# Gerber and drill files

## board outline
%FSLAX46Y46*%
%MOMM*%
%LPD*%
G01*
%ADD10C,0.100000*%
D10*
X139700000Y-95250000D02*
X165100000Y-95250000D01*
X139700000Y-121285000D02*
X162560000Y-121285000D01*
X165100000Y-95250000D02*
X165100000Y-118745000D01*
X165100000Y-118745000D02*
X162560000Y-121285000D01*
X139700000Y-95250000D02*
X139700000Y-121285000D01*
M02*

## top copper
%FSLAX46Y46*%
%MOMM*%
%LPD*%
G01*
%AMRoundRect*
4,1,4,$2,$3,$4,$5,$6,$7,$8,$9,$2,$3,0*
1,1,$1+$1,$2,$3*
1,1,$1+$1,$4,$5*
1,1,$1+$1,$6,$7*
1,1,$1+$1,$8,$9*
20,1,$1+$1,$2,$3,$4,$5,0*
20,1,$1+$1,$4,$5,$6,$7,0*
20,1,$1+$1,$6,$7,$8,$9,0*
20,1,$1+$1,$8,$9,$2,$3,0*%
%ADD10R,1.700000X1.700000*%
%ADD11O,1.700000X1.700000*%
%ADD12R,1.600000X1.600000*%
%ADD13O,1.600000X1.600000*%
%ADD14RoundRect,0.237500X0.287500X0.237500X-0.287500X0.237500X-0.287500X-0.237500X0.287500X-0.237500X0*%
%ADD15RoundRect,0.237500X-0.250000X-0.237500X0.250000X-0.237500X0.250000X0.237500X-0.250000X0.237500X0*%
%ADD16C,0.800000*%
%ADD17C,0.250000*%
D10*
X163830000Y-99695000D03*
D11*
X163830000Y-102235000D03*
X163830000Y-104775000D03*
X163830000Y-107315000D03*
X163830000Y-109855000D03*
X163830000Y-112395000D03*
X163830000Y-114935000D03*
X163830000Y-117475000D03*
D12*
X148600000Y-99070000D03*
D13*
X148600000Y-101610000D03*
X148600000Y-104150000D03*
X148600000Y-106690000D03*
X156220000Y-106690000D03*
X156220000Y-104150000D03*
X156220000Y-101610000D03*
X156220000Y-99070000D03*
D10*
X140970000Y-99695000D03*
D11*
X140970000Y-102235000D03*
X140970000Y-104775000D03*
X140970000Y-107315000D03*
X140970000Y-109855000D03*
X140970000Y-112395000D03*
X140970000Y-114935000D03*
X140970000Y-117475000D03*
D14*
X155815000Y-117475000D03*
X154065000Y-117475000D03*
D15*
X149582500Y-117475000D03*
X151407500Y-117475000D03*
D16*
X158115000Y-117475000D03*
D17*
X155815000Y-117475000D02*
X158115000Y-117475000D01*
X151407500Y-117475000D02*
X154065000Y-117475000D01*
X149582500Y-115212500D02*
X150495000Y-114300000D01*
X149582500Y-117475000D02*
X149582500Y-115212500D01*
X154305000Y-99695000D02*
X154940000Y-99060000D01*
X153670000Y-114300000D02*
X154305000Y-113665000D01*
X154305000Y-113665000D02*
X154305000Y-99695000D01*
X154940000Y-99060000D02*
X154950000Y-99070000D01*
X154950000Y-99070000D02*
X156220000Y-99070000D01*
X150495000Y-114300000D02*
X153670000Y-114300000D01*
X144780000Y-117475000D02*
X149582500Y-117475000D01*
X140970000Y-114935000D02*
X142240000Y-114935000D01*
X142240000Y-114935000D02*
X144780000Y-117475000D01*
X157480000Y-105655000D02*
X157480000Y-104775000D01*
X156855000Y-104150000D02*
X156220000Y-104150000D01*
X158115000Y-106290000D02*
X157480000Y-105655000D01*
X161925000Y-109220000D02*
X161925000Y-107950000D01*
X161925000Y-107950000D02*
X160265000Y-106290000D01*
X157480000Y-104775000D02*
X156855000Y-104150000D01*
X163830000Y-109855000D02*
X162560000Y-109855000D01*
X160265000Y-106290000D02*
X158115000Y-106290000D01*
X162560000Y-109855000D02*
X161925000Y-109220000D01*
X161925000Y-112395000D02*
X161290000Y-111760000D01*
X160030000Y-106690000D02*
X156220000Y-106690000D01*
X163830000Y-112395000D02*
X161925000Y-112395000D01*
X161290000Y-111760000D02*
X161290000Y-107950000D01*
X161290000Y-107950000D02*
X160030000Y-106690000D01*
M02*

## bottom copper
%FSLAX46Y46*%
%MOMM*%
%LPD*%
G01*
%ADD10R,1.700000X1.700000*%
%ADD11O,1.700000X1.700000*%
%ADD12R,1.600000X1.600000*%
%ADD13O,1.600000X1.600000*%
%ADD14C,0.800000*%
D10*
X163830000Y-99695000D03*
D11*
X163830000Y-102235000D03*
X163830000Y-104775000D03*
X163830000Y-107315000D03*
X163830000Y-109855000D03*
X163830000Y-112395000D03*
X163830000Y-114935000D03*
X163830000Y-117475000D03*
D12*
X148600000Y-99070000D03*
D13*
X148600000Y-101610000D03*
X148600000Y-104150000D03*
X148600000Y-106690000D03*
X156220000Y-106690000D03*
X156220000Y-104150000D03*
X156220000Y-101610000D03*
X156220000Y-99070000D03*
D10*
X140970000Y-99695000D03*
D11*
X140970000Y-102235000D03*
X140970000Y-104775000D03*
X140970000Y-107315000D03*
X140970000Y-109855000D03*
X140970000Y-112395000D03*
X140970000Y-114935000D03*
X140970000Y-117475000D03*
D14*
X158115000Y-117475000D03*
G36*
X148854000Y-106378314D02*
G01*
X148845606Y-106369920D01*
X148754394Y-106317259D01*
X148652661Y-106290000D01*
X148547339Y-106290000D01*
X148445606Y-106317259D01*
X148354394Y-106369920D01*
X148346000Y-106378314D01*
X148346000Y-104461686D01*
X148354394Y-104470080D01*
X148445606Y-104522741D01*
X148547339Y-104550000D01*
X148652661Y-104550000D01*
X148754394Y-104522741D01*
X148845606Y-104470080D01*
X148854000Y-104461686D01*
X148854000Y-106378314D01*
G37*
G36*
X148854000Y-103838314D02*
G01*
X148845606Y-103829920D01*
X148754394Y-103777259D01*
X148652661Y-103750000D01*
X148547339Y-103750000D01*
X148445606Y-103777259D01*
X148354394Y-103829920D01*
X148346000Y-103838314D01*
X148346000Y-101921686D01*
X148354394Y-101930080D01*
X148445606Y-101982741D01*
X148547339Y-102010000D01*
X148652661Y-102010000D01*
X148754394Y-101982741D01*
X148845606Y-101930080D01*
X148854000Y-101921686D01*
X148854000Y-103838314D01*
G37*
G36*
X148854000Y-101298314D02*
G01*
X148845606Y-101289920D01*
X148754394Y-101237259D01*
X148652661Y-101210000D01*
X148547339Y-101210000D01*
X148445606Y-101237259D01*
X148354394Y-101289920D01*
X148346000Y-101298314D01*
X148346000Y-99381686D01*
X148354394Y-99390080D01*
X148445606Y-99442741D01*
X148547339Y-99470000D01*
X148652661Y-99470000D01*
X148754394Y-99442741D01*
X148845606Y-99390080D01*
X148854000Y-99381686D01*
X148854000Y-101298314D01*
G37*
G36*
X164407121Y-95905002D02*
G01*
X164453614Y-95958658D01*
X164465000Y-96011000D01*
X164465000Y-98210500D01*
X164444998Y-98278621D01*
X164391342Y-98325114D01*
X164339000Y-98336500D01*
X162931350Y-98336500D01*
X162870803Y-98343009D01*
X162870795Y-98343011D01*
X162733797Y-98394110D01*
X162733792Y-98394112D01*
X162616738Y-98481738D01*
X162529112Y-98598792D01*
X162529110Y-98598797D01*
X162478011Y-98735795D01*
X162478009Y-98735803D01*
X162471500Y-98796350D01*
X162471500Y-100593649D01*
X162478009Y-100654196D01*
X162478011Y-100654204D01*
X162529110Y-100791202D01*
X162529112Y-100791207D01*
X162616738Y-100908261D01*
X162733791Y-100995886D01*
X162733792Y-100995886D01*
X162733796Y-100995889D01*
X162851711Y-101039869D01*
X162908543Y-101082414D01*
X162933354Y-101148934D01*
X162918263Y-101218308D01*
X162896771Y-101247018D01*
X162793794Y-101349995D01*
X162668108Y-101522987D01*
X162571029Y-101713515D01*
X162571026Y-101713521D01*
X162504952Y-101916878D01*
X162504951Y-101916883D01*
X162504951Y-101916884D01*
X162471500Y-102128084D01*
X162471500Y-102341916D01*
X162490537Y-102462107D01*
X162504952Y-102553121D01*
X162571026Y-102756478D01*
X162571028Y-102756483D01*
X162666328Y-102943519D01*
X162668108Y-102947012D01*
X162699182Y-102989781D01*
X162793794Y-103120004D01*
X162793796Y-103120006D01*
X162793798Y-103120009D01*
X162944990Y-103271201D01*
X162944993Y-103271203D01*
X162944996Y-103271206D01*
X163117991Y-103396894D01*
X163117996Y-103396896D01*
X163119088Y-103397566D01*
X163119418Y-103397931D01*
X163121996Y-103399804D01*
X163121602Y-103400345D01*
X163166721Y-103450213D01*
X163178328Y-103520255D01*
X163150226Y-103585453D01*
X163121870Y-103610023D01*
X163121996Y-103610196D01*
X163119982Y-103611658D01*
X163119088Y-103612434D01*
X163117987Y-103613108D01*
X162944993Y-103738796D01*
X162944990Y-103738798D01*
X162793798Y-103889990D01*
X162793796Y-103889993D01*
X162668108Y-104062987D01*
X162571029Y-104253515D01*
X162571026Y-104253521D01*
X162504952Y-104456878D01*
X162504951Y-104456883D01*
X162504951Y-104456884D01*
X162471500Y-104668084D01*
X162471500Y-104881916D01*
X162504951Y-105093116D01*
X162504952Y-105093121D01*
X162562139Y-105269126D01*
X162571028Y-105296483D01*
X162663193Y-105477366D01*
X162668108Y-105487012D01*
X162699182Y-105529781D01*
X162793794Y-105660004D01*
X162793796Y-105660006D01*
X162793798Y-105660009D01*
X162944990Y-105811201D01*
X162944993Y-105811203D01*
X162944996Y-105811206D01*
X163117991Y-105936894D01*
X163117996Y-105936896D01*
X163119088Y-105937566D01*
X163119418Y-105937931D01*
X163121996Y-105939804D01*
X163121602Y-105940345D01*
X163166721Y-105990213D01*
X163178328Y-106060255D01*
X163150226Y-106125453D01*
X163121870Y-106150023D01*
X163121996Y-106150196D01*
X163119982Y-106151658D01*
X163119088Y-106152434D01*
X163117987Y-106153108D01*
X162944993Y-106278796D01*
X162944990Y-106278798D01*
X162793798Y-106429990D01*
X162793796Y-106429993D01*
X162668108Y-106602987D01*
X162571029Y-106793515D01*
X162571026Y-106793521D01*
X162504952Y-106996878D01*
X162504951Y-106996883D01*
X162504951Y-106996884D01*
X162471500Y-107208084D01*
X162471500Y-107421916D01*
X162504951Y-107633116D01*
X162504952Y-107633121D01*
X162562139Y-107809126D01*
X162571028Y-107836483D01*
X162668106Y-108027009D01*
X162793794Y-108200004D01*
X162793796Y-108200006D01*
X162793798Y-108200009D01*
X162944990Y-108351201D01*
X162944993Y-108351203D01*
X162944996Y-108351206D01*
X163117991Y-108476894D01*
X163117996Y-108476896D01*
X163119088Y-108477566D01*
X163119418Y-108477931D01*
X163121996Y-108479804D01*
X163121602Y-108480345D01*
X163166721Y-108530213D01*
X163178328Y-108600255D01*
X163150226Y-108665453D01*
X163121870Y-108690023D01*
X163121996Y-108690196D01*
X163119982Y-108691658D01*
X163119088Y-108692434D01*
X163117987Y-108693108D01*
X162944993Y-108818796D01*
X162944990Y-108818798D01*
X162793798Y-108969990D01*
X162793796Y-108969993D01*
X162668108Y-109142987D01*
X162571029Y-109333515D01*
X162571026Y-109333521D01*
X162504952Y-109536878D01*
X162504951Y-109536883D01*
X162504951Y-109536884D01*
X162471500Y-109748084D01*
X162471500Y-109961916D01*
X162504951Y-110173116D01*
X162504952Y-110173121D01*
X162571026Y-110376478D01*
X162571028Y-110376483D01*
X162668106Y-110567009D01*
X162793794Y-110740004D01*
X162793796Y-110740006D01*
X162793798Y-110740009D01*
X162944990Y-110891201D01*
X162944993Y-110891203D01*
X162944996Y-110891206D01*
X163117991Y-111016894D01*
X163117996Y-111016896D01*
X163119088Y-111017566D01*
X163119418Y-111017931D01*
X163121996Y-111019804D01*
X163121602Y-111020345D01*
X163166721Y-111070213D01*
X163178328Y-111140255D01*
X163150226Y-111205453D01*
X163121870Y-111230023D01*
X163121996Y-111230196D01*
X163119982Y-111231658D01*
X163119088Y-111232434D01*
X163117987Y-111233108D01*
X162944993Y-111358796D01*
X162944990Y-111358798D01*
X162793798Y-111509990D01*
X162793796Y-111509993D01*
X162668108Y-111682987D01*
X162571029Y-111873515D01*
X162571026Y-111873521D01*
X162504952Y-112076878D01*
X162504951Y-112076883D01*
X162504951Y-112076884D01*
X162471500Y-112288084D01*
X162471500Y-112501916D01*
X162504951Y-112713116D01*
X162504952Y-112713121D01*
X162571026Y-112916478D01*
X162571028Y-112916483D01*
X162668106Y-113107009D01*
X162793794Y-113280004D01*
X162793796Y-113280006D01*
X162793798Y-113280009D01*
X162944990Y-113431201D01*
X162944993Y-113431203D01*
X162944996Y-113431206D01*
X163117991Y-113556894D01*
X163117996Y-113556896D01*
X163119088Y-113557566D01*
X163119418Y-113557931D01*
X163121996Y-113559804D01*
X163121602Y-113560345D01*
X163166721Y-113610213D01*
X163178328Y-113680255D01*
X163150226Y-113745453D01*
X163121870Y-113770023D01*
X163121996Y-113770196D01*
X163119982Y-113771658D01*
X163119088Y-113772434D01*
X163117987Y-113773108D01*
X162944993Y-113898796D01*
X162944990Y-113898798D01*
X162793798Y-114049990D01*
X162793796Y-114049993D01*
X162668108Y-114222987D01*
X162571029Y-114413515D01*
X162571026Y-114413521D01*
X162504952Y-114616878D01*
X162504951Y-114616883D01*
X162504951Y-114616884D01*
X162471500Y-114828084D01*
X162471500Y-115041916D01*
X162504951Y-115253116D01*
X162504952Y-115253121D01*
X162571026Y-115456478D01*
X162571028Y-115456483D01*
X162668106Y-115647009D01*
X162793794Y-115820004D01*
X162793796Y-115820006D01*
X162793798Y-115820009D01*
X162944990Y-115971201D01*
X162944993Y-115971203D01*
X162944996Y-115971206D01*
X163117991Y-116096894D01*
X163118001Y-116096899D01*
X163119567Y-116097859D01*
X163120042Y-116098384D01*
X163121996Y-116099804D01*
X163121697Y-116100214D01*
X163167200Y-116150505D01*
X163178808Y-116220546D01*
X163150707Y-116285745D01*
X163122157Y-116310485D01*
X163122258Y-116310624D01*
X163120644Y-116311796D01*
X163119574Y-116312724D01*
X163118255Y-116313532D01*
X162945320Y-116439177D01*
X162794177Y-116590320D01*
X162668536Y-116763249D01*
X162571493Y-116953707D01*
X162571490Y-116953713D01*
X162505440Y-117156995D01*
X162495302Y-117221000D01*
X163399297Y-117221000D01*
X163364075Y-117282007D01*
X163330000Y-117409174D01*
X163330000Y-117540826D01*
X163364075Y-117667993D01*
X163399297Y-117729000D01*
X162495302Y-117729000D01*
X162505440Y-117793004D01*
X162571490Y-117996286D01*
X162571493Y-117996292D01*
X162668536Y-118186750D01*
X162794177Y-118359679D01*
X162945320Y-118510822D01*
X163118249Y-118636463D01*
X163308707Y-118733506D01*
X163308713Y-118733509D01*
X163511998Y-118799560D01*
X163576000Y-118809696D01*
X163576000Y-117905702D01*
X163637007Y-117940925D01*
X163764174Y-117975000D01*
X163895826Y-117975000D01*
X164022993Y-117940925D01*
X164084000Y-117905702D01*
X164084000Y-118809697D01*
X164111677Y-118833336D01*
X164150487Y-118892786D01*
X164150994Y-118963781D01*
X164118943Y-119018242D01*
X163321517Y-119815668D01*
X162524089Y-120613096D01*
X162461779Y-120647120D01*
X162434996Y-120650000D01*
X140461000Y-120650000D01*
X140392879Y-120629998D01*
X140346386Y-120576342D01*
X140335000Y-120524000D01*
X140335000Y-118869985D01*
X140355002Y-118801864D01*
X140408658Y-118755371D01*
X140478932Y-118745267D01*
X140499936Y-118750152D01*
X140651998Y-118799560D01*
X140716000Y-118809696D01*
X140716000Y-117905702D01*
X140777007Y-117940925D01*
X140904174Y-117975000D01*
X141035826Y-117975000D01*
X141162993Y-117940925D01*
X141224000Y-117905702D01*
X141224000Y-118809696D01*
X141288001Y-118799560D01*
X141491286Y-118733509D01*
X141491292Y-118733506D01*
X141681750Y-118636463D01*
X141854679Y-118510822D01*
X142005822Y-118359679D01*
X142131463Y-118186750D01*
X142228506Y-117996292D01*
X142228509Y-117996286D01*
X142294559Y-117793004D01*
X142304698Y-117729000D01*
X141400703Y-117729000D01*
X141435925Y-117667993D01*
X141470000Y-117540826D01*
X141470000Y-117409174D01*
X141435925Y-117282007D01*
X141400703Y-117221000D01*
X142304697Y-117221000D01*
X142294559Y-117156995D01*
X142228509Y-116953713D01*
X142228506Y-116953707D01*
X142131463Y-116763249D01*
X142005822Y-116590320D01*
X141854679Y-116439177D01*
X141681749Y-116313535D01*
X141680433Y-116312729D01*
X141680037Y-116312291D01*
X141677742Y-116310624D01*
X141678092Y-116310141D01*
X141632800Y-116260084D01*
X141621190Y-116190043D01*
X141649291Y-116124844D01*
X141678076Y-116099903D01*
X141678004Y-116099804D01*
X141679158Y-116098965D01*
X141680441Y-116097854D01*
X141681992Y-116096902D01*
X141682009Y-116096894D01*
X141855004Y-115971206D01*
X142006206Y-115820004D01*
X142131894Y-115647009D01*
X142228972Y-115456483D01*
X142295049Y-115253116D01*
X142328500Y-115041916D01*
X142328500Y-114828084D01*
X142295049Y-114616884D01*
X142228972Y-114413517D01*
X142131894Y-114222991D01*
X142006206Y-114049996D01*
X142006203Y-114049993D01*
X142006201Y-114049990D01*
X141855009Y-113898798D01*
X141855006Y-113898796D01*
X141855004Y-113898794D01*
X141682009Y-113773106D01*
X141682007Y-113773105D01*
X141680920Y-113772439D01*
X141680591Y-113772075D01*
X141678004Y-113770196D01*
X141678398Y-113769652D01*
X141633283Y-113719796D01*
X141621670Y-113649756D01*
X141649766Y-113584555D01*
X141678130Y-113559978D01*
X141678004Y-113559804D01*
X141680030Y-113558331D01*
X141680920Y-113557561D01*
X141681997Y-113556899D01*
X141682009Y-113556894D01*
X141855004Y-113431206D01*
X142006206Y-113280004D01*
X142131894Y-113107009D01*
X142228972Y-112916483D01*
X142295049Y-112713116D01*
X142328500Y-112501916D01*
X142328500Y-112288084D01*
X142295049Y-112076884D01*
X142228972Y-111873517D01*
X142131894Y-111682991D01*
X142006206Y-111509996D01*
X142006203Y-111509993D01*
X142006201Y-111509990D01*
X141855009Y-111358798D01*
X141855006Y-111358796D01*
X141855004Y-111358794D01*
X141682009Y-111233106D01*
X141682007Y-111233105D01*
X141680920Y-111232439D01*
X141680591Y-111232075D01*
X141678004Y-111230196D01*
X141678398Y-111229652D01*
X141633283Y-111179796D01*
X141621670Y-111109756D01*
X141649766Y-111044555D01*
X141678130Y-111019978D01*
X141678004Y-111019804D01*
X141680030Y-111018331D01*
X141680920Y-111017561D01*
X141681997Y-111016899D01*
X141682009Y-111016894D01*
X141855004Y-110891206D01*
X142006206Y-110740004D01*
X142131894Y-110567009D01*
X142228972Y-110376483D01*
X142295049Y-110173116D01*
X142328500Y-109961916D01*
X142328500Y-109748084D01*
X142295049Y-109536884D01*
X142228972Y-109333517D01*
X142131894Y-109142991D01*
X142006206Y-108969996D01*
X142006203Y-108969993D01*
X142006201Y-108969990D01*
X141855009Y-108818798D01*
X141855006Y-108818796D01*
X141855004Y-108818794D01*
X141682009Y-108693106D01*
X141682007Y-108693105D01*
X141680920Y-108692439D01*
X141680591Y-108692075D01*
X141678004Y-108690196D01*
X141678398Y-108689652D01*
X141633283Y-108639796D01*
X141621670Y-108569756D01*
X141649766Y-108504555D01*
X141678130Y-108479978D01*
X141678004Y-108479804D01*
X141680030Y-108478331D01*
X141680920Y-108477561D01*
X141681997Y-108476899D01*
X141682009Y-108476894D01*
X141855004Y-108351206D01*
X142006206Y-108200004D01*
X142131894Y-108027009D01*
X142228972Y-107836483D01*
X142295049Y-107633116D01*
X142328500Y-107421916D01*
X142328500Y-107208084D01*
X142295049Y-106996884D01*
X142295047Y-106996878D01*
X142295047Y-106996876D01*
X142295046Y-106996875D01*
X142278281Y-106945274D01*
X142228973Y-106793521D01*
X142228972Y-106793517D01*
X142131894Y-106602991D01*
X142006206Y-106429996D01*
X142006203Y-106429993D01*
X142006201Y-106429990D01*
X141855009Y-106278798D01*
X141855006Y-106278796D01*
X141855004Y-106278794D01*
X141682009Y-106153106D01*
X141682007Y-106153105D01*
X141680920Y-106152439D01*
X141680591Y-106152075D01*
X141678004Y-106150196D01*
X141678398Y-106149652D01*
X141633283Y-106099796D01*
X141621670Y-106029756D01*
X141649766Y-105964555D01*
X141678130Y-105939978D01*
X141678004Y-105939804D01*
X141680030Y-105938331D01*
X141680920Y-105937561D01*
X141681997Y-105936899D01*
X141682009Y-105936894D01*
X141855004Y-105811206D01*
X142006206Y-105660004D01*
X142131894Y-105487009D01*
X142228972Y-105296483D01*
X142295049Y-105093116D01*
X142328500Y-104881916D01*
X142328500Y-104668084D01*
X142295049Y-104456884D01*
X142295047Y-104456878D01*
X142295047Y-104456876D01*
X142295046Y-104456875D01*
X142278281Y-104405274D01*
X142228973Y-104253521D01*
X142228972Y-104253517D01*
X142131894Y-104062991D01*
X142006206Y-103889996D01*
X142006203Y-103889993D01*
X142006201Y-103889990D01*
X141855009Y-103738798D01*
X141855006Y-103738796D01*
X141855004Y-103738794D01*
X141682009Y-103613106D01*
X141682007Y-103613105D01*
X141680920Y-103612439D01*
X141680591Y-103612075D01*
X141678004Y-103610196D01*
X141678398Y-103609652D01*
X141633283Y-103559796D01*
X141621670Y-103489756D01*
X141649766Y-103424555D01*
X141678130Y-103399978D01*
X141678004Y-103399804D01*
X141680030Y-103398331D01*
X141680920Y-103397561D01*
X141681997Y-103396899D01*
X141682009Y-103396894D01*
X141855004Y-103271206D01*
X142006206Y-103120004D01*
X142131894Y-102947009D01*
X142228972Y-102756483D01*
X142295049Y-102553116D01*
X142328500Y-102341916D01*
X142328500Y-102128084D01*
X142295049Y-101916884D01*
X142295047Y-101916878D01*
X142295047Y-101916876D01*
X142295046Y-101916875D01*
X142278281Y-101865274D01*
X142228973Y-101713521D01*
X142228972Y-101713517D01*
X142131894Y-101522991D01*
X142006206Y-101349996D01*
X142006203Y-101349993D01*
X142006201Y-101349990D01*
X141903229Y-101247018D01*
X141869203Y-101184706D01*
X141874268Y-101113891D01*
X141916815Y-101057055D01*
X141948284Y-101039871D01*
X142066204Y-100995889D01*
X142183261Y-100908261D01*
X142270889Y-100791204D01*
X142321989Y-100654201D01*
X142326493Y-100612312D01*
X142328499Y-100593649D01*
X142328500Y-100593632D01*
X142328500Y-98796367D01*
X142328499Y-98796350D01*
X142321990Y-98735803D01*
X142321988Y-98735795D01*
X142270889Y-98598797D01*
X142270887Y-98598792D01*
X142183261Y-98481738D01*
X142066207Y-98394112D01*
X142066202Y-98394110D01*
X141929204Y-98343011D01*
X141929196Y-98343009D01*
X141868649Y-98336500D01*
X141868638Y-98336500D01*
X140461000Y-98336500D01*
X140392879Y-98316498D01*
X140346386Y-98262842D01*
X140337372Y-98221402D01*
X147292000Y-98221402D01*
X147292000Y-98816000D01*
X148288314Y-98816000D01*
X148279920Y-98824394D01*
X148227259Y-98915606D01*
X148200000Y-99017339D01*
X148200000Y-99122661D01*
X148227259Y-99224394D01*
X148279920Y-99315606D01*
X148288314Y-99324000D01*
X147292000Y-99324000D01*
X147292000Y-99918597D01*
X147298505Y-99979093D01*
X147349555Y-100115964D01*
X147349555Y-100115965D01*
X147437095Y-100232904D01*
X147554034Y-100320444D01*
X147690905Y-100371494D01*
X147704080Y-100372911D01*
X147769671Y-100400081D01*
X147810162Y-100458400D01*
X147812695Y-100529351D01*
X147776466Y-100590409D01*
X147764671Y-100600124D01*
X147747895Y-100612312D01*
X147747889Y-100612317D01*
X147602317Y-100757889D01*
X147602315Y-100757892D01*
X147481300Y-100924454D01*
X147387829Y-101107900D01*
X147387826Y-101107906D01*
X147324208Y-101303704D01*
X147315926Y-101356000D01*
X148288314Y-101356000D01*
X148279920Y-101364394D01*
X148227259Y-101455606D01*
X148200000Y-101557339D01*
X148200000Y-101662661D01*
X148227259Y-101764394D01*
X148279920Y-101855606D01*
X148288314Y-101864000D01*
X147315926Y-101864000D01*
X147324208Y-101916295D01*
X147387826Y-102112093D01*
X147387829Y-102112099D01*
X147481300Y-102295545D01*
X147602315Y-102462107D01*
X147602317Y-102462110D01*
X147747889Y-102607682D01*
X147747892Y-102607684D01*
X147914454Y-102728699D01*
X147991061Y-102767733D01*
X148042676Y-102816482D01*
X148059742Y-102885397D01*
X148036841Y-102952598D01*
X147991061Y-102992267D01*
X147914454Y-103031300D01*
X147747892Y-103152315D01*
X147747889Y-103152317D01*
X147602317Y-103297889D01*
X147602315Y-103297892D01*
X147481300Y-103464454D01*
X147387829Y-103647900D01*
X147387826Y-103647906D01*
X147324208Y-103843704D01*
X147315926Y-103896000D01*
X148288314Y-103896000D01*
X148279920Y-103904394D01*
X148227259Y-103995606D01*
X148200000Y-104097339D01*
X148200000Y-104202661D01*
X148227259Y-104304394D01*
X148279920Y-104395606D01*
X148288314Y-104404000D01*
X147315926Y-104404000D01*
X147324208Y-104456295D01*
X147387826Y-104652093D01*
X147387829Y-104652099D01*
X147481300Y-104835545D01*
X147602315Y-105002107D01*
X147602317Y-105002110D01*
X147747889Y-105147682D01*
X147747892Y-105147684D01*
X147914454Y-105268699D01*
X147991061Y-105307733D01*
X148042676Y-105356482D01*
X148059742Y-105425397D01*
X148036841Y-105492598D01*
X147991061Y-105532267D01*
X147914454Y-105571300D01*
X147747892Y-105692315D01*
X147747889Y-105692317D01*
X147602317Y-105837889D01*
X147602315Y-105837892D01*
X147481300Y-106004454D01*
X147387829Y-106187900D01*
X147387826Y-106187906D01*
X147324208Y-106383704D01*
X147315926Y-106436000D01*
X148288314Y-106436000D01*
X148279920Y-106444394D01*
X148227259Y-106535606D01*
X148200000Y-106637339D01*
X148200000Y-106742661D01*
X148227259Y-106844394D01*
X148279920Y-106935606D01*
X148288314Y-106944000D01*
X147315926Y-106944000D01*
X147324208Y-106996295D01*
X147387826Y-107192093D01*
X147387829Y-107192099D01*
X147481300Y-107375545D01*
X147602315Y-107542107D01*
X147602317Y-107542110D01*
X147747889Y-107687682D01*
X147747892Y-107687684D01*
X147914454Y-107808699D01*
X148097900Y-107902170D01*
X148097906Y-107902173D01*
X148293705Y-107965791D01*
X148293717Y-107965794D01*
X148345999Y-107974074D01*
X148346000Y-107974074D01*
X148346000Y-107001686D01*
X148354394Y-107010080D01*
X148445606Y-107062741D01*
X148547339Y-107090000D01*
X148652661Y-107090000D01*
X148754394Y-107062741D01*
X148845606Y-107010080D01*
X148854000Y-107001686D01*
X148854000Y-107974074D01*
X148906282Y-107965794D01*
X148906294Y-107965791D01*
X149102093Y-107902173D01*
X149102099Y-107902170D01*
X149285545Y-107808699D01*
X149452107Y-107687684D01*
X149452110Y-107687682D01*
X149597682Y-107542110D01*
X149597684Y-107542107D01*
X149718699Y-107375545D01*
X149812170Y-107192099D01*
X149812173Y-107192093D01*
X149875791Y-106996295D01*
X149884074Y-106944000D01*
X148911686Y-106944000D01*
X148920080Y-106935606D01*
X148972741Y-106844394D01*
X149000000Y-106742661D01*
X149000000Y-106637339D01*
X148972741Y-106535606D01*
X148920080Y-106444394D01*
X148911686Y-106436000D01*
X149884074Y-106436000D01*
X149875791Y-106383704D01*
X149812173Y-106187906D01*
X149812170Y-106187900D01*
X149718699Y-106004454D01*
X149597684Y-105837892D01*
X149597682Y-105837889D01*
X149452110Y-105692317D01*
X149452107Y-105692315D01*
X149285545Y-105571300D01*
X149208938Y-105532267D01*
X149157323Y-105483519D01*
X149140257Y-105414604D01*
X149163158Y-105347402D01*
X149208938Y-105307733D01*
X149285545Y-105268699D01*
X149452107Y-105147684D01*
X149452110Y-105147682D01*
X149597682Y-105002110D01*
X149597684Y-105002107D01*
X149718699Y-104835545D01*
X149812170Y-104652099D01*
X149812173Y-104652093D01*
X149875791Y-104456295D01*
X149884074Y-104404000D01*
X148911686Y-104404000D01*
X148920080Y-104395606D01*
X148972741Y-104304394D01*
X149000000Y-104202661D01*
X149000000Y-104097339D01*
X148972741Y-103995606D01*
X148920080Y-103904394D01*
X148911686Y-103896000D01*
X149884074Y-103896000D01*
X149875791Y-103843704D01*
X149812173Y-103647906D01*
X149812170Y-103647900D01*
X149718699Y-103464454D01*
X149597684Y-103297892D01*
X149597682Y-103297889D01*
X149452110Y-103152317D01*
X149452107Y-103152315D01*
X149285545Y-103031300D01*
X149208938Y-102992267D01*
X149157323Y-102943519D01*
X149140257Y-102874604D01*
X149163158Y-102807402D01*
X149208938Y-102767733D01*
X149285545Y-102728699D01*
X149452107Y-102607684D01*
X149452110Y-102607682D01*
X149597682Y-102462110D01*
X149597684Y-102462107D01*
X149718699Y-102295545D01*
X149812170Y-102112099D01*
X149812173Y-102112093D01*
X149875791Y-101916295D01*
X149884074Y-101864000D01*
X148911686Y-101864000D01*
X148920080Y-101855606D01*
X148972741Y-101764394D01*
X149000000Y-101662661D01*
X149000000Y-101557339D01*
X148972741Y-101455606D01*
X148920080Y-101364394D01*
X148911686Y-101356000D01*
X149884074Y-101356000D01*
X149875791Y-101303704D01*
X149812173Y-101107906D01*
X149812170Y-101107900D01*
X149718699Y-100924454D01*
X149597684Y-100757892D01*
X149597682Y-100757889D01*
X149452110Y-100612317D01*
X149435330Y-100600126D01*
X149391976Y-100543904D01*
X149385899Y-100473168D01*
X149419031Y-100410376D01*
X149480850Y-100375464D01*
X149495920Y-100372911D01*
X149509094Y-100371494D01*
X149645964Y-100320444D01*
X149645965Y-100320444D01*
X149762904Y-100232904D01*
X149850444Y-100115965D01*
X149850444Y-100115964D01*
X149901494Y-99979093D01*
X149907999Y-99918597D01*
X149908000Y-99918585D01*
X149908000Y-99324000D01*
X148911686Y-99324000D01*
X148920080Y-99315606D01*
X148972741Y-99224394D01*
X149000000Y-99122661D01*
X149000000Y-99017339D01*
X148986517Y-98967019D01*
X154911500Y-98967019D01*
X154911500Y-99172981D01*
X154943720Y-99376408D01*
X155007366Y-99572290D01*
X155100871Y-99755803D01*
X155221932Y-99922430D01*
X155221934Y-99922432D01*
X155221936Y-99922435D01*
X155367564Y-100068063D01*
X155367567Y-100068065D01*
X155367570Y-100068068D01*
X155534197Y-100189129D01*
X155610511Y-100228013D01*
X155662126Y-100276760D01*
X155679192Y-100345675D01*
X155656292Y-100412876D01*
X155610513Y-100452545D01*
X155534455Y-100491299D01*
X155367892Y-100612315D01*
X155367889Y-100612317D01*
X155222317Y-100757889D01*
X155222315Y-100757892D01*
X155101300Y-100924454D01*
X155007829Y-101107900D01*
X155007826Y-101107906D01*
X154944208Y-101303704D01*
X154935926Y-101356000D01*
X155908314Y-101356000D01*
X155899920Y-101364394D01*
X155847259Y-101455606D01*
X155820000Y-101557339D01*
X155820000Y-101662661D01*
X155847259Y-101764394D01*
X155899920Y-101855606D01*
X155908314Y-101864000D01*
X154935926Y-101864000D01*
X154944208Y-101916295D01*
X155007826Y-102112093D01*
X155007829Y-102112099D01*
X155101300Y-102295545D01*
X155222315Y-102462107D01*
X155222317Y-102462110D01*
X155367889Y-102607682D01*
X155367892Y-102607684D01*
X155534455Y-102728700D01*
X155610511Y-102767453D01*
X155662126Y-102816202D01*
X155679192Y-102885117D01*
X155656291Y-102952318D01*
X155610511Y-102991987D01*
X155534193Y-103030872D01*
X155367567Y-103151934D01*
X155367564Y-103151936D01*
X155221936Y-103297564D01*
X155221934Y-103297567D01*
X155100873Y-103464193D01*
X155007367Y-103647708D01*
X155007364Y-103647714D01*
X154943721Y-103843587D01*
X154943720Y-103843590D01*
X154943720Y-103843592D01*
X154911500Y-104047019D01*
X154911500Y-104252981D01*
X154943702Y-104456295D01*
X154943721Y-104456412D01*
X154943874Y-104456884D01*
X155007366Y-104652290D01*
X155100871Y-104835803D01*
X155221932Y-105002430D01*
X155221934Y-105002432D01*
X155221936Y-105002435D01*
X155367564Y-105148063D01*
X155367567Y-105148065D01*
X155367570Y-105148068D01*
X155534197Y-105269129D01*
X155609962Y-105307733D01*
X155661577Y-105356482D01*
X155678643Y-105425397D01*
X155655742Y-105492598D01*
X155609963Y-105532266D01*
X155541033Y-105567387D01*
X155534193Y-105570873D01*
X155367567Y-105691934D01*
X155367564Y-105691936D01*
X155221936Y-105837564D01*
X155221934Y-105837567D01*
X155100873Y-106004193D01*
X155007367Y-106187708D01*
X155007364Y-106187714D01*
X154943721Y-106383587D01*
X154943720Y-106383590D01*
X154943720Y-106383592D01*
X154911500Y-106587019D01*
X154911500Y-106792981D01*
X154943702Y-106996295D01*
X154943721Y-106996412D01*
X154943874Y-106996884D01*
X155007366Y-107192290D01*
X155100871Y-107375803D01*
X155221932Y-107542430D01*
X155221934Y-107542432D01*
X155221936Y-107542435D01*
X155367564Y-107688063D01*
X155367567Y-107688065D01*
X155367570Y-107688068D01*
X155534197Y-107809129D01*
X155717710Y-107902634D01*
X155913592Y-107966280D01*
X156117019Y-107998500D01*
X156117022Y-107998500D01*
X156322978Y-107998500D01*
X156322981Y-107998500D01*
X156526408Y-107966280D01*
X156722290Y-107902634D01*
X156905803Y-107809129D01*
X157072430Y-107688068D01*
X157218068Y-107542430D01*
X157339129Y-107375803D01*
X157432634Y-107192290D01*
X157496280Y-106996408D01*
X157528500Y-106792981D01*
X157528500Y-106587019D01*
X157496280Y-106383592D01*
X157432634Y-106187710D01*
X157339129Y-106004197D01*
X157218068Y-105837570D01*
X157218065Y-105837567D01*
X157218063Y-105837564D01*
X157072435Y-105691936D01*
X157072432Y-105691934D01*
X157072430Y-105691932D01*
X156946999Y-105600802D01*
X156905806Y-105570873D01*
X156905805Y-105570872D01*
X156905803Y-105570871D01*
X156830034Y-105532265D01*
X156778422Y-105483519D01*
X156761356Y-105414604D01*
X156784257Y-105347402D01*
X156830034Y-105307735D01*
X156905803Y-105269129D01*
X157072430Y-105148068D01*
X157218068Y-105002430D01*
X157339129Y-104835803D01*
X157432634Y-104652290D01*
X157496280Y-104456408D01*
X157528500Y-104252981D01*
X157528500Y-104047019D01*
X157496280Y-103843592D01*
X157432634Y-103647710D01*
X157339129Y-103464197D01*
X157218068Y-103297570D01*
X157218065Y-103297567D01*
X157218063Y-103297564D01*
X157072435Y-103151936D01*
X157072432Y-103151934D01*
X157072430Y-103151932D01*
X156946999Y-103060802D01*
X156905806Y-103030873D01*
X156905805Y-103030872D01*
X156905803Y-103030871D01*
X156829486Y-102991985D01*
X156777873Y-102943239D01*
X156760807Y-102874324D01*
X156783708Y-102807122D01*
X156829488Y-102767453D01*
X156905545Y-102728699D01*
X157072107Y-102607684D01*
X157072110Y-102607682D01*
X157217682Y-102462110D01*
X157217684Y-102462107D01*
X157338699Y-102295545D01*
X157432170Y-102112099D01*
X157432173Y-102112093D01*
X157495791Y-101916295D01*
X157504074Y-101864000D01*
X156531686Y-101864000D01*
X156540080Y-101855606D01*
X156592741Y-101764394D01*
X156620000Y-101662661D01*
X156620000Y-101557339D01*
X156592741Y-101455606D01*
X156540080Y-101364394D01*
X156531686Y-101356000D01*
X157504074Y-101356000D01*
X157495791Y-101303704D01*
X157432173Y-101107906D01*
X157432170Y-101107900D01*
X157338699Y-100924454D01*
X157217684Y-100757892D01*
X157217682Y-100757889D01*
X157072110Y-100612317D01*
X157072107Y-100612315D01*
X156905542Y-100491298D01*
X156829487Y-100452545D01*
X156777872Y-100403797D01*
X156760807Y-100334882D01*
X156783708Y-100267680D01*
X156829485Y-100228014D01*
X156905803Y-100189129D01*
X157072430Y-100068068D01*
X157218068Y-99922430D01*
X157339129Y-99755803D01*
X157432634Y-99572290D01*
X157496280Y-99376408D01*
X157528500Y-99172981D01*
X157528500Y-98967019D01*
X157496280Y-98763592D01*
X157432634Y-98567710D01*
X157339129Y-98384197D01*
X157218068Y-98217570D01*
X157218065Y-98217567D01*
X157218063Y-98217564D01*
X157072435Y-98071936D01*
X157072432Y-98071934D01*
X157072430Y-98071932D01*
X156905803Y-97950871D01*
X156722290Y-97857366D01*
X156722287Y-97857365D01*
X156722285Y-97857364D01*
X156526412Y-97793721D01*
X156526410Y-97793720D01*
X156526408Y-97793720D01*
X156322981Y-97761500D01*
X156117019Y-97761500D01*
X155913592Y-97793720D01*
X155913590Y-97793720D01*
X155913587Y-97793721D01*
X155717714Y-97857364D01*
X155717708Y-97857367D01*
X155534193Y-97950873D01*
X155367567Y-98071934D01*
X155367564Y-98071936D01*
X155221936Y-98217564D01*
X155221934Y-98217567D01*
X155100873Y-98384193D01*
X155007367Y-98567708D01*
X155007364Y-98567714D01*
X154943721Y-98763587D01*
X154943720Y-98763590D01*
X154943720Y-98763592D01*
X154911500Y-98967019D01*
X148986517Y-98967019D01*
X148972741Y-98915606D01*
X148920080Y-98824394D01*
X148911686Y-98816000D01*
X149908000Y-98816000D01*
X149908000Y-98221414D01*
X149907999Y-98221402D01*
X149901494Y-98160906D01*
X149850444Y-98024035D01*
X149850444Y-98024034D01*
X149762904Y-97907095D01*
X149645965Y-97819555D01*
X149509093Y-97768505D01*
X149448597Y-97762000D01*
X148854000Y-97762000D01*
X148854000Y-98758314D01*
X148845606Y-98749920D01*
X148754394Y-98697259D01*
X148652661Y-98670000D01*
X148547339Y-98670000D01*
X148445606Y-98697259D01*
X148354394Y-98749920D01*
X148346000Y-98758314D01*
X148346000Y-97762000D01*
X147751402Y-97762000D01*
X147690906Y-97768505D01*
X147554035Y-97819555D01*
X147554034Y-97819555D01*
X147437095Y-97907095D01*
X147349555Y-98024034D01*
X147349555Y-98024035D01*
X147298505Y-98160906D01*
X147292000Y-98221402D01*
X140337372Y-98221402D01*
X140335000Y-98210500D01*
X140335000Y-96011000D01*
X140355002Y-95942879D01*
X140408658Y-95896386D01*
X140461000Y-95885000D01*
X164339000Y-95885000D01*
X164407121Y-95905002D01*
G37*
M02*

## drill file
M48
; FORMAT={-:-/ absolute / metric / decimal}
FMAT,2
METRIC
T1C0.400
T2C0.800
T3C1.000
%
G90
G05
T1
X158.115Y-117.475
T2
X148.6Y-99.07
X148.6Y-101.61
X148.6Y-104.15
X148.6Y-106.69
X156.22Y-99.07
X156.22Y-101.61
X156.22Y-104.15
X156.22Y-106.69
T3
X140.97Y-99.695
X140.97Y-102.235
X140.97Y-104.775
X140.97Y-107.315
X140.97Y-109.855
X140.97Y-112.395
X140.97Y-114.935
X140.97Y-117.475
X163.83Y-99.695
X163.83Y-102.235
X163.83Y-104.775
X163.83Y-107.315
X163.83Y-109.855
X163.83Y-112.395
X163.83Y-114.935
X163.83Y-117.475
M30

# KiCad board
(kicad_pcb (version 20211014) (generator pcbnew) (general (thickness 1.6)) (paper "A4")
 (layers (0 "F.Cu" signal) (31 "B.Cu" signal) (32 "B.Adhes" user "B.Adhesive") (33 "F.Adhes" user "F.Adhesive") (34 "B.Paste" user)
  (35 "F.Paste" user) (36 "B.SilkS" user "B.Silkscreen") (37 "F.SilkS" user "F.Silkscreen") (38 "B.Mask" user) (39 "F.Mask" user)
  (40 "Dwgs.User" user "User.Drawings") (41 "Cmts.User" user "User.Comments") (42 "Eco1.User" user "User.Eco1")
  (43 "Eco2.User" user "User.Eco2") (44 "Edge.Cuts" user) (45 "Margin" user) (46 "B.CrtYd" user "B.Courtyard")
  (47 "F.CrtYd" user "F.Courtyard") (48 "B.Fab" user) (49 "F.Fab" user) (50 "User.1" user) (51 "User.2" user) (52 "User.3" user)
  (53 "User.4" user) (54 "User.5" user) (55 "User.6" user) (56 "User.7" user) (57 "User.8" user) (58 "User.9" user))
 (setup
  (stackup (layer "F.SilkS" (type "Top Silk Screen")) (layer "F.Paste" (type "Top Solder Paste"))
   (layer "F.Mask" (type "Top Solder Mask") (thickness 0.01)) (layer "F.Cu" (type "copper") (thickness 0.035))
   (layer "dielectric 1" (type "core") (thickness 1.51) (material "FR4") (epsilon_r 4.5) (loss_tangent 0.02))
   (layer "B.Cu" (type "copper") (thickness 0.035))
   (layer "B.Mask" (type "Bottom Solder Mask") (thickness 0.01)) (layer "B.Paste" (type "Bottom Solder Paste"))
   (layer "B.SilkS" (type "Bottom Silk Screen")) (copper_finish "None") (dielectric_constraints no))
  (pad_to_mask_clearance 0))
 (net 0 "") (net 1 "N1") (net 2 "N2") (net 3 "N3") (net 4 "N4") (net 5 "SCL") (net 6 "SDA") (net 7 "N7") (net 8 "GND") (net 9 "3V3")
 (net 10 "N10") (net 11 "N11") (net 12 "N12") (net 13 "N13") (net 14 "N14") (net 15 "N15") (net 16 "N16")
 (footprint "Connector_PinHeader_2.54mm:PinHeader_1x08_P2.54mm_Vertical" (layer "F.Cu") (at 163.83 99.695)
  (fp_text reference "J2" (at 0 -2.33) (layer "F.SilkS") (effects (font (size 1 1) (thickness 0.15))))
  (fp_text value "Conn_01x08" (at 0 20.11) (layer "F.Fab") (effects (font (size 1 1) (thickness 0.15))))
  (pad "1" thru_hole rect (at 0 0) (size 1.7 1.7) (drill 1) (layers *.Cu *.Mask) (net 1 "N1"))
  (pad "2" thru_hole oval (at 0 2.54) (size 1.7 1.7) (drill 1) (layers *.Cu *.Mask) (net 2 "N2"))
  (pad "3" thru_hole oval (at 0 5.08) (size 1.7 1.7) (drill 1) (layers *.Cu *.Mask) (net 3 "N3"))
  (pad "4" thru_hole oval (at 0 7.62) (size 1.7 1.7) (drill 1) (layers *.Cu *.Mask) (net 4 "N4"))
  (pad "5" thru_hole oval (at 0 10.16) (size 1.7 1.7) (drill 1) (layers *.Cu *.Mask) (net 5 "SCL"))
  (pad "6" thru_hole oval (at 0 12.7) (size 1.7 1.7) (drill 1) (layers *.Cu *.Mask) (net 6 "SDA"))
  (pad "7" thru_hole oval (at 0 15.24) (size 1.7 1.7) (drill 1) (layers *.Cu *.Mask) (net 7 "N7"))
  (pad "8" thru_hole oval (at 0 17.78) (size 1.7 1.7) (drill 1) (layers *.Cu *.Mask) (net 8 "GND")))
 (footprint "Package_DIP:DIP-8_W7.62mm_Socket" (layer "F.Cu") (at 148.6 99.07)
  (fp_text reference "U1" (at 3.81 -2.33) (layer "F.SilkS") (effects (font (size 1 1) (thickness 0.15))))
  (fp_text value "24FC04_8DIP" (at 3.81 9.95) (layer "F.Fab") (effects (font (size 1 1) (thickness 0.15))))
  (pad "1" thru_hole rect (at 0 0) (size 1.6 1.6) (drill 0.8) (layers *.Cu *.Mask) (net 8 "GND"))
  (pad "2" thru_hole oval (at 0 2.54) (size 1.6 1.6) (drill 0.8) (layers *.Cu *.Mask) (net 8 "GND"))
  (pad "3" thru_hole oval (at 0 5.08) (size 1.6 1.6) (drill 0.8) (layers *.Cu *.Mask) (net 8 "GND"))
  (pad "4" thru_hole oval (at 0 7.62) (size 1.6 1.6) (drill 0.8) (layers *.Cu *.Mask) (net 8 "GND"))
  (pad "5" thru_hole oval (at 7.62 7.62) (size 1.6 1.6) (drill 0.8) (layers *.Cu *.Mask) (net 6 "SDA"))
  (pad "6" thru_hole oval (at 7.62 5.08) (size 1.6 1.6) (drill 0.8) (layers *.Cu *.Mask) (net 5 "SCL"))
  (pad "7" thru_hole oval (at 7.62 2.54) (size 1.6 1.6) (drill 0.8) (layers *.Cu *.Mask) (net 8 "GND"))
  (pad "8" thru_hole oval (at 7.62 0) (size 1.6 1.6) (drill 0.8) (layers *.Cu *.Mask) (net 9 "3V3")))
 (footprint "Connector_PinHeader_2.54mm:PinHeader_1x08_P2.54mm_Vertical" (layer "F.Cu") (at 140.97 99.695)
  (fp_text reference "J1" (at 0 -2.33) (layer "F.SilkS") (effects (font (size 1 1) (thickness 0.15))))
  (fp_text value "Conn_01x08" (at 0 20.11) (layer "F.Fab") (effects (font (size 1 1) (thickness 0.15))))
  (pad "1" thru_hole rect (at 0 0) (size 1.7 1.7) (drill 1) (layers *.Cu *.Mask) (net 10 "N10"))
  (pad "2" thru_hole oval (at 0 2.54) (size 1.7 1.7) (drill 1) (layers *.Cu *.Mask) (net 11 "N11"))
  (pad "3" thru_hole oval (at 0 5.08) (size 1.7 1.7) (drill 1) (layers *.Cu *.Mask) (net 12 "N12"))
  (pad "4" thru_hole oval (at 0 7.62) (size 1.7 1.7) (drill 1) (layers *.Cu *.Mask) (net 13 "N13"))
  (pad "5" thru_hole oval (at 0 10.16) (size 1.7 1.7) (drill 1) (layers *.Cu *.Mask) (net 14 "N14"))
  (pad "6" thru_hole oval (at 0 12.7) (size 1.7 1.7) (drill 1) (layers *.Cu *.Mask) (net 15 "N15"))
  (pad "7" thru_hole oval (at 0 15.24) (size 1.7 1.7) (drill 1) (layers *.Cu *.Mask) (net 9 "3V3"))
  (pad "8" thru_hole oval (at 0 17.78) (size 1.7 1.7) (drill 1) (layers *.Cu *.Mask) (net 8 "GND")))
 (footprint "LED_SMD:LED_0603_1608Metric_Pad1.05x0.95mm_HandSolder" (layer "F.Cu") (at 154.94 117.475 180)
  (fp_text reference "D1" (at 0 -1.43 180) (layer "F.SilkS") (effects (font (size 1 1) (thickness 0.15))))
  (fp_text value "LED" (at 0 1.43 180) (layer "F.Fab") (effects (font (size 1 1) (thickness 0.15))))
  (pad "1" smd roundrect (at -0.875 0 180) (size 1.05 0.95) (layers "F.Cu" "F.Paste" "F.Mask") (roundrect_rratio 0.25) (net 8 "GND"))
  (pad "2" smd roundrect (at 0.875 0 180) (size 1.05 0.95) (layers "F.Cu" "F.Paste" "F.Mask") (roundrect_rratio 0.25) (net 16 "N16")))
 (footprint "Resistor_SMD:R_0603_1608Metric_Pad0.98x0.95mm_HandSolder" (layer "F.Cu") (at 150.495 117.475)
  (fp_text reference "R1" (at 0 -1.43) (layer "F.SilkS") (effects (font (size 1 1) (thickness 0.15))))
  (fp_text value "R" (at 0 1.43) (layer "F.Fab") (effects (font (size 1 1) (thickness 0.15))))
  (pad "1" smd roundrect (at -0.9125 0) (size 0.975 0.95) (layers "F.Cu" "F.Paste" "F.Mask") (roundrect_rratio 0.25) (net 9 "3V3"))
  (pad "2" smd roundrect (at 0.9125 0) (size 0.975 0.95) (layers "F.Cu" "F.Paste" "F.Mask") (roundrect_rratio 0.25) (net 16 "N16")))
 (gr_line (start 139.7 95.25) (end 165.1 95.25) (layer "Edge.Cuts") (width 0.1))
 (gr_line (start 139.7 121.285) (end 162.56 121.285) (layer "Edge.Cuts") (width 0.1))
 (gr_line (start 165.1 95.25) (end 165.1 118.745) (layer "Edge.Cuts") (width 0.1))
 (gr_line (start 165.1 118.745) (end 162.56 121.285) (layer "Edge.Cuts") (width 0.1))
 (gr_line (start 139.7 95.25) (end 139.7 121.285) (layer "Edge.Cuts") (width 0.1))
 (segment (start 155.815 117.475) (end 158.115 117.475) (width 0.25) (layer "F.Cu") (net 8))
 (via (at 158.115 117.475) (size 0.8) (drill 0.4) (layers "F.Cu" "B.Cu") (free) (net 8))
 (segment (start 151.4075 117.475) (end 154.065 117.475) (width 0.25) (layer "F.Cu") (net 16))
 (segment (start 149.5825 115.2125) (end 150.495 114.3) (width 0.25) (layer "F.Cu") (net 9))
 (segment (start 149.5825 117.475) (end 149.5825 115.2125) (width 0.25) (layer "F.Cu") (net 9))
 (segment (start 154.305 99.695) (end 154.94 99.06) (width 0.25) (layer "F.Cu") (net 9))
 (segment (start 153.67 114.3) (end 154.305 113.665) (width 0.25) (layer "F.Cu") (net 9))
 (segment (start 154.305 113.665) (end 154.305 99.695) (width 0.25) (layer "F.Cu") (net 9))
 (segment (start 154.94 99.06) (end 154.95 99.07) (width 0.25) (layer "F.Cu") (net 9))
 (segment (start 154.95 99.07) (end 156.22 99.07) (width 0.25) (layer "F.Cu") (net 9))
 (segment (start 150.495 114.3) (end 153.67 114.3) (width 0.25) (layer "F.Cu") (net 9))
 (segment (start 144.78 117.475) (end 149.5825 117.475) (width 0.25) (layer "F.Cu") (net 9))
 (segment (start 140.97 114.935) (end 142.24 114.935) (width 0.25) (layer "F.Cu") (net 9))
 (segment (start 142.24 114.935) (end 144.78 117.475) (width 0.25) (layer "F.Cu") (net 9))
 (segment (start 157.48 105.655) (end 157.48 104.775) (width 0.25) (layer "F.Cu") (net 5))
 (segment (start 156.855 104.15) (end 156.22 104.15) (width 0.25) (layer "F.Cu") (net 5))
 (segment (start 158.115 106.29) (end 157.48 105.655) (width 0.25) (layer "F.Cu") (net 5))
 (segment (start 161.925 109.22) (end 161.925 107.95) (width 0.25) (layer "F.Cu") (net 5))
 (segment (start 161.925 107.95) (end 160.265 106.29) (width 0.25) (layer "F.Cu") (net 5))
 (segment (start 157.48 104.775) (end 156.855 104.15) (width 0.25) (layer "F.Cu") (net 5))
 (segment (start 163.83 109.855) (end 162.56 109.855) (width 0.25) (layer "F.Cu") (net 5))
 (segment (start 160.265 106.29) (end 158.115 106.29) (width 0.25) (layer "F.Cu") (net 5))
 (segment (start 162.56 109.855) (end 161.925 109.22) (width 0.25) (layer "F.Cu") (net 5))
 (segment (start 161.925 112.395) (end 161.29 111.76) (width 0.25) (layer "F.Cu") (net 6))
 (segment (start 160.03 106.69) (end 156.22 106.69) (width 0.25) (layer "F.Cu") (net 6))
 (segment (start 163.83 112.395) (end 161.925 112.395) (width 0.25) (layer "F.Cu") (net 6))
 (segment (start 161.29 111.76) (end 161.29 107.95) (width 0.25) (layer "F.Cu") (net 6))
 (segment (start 161.29 107.95) (end 160.03 106.69) (width 0.25) (layer "F.Cu") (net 6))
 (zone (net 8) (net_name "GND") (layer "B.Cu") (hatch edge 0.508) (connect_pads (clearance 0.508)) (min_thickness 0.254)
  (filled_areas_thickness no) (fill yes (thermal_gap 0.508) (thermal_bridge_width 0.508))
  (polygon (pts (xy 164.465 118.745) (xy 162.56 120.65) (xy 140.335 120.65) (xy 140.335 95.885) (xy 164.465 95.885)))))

